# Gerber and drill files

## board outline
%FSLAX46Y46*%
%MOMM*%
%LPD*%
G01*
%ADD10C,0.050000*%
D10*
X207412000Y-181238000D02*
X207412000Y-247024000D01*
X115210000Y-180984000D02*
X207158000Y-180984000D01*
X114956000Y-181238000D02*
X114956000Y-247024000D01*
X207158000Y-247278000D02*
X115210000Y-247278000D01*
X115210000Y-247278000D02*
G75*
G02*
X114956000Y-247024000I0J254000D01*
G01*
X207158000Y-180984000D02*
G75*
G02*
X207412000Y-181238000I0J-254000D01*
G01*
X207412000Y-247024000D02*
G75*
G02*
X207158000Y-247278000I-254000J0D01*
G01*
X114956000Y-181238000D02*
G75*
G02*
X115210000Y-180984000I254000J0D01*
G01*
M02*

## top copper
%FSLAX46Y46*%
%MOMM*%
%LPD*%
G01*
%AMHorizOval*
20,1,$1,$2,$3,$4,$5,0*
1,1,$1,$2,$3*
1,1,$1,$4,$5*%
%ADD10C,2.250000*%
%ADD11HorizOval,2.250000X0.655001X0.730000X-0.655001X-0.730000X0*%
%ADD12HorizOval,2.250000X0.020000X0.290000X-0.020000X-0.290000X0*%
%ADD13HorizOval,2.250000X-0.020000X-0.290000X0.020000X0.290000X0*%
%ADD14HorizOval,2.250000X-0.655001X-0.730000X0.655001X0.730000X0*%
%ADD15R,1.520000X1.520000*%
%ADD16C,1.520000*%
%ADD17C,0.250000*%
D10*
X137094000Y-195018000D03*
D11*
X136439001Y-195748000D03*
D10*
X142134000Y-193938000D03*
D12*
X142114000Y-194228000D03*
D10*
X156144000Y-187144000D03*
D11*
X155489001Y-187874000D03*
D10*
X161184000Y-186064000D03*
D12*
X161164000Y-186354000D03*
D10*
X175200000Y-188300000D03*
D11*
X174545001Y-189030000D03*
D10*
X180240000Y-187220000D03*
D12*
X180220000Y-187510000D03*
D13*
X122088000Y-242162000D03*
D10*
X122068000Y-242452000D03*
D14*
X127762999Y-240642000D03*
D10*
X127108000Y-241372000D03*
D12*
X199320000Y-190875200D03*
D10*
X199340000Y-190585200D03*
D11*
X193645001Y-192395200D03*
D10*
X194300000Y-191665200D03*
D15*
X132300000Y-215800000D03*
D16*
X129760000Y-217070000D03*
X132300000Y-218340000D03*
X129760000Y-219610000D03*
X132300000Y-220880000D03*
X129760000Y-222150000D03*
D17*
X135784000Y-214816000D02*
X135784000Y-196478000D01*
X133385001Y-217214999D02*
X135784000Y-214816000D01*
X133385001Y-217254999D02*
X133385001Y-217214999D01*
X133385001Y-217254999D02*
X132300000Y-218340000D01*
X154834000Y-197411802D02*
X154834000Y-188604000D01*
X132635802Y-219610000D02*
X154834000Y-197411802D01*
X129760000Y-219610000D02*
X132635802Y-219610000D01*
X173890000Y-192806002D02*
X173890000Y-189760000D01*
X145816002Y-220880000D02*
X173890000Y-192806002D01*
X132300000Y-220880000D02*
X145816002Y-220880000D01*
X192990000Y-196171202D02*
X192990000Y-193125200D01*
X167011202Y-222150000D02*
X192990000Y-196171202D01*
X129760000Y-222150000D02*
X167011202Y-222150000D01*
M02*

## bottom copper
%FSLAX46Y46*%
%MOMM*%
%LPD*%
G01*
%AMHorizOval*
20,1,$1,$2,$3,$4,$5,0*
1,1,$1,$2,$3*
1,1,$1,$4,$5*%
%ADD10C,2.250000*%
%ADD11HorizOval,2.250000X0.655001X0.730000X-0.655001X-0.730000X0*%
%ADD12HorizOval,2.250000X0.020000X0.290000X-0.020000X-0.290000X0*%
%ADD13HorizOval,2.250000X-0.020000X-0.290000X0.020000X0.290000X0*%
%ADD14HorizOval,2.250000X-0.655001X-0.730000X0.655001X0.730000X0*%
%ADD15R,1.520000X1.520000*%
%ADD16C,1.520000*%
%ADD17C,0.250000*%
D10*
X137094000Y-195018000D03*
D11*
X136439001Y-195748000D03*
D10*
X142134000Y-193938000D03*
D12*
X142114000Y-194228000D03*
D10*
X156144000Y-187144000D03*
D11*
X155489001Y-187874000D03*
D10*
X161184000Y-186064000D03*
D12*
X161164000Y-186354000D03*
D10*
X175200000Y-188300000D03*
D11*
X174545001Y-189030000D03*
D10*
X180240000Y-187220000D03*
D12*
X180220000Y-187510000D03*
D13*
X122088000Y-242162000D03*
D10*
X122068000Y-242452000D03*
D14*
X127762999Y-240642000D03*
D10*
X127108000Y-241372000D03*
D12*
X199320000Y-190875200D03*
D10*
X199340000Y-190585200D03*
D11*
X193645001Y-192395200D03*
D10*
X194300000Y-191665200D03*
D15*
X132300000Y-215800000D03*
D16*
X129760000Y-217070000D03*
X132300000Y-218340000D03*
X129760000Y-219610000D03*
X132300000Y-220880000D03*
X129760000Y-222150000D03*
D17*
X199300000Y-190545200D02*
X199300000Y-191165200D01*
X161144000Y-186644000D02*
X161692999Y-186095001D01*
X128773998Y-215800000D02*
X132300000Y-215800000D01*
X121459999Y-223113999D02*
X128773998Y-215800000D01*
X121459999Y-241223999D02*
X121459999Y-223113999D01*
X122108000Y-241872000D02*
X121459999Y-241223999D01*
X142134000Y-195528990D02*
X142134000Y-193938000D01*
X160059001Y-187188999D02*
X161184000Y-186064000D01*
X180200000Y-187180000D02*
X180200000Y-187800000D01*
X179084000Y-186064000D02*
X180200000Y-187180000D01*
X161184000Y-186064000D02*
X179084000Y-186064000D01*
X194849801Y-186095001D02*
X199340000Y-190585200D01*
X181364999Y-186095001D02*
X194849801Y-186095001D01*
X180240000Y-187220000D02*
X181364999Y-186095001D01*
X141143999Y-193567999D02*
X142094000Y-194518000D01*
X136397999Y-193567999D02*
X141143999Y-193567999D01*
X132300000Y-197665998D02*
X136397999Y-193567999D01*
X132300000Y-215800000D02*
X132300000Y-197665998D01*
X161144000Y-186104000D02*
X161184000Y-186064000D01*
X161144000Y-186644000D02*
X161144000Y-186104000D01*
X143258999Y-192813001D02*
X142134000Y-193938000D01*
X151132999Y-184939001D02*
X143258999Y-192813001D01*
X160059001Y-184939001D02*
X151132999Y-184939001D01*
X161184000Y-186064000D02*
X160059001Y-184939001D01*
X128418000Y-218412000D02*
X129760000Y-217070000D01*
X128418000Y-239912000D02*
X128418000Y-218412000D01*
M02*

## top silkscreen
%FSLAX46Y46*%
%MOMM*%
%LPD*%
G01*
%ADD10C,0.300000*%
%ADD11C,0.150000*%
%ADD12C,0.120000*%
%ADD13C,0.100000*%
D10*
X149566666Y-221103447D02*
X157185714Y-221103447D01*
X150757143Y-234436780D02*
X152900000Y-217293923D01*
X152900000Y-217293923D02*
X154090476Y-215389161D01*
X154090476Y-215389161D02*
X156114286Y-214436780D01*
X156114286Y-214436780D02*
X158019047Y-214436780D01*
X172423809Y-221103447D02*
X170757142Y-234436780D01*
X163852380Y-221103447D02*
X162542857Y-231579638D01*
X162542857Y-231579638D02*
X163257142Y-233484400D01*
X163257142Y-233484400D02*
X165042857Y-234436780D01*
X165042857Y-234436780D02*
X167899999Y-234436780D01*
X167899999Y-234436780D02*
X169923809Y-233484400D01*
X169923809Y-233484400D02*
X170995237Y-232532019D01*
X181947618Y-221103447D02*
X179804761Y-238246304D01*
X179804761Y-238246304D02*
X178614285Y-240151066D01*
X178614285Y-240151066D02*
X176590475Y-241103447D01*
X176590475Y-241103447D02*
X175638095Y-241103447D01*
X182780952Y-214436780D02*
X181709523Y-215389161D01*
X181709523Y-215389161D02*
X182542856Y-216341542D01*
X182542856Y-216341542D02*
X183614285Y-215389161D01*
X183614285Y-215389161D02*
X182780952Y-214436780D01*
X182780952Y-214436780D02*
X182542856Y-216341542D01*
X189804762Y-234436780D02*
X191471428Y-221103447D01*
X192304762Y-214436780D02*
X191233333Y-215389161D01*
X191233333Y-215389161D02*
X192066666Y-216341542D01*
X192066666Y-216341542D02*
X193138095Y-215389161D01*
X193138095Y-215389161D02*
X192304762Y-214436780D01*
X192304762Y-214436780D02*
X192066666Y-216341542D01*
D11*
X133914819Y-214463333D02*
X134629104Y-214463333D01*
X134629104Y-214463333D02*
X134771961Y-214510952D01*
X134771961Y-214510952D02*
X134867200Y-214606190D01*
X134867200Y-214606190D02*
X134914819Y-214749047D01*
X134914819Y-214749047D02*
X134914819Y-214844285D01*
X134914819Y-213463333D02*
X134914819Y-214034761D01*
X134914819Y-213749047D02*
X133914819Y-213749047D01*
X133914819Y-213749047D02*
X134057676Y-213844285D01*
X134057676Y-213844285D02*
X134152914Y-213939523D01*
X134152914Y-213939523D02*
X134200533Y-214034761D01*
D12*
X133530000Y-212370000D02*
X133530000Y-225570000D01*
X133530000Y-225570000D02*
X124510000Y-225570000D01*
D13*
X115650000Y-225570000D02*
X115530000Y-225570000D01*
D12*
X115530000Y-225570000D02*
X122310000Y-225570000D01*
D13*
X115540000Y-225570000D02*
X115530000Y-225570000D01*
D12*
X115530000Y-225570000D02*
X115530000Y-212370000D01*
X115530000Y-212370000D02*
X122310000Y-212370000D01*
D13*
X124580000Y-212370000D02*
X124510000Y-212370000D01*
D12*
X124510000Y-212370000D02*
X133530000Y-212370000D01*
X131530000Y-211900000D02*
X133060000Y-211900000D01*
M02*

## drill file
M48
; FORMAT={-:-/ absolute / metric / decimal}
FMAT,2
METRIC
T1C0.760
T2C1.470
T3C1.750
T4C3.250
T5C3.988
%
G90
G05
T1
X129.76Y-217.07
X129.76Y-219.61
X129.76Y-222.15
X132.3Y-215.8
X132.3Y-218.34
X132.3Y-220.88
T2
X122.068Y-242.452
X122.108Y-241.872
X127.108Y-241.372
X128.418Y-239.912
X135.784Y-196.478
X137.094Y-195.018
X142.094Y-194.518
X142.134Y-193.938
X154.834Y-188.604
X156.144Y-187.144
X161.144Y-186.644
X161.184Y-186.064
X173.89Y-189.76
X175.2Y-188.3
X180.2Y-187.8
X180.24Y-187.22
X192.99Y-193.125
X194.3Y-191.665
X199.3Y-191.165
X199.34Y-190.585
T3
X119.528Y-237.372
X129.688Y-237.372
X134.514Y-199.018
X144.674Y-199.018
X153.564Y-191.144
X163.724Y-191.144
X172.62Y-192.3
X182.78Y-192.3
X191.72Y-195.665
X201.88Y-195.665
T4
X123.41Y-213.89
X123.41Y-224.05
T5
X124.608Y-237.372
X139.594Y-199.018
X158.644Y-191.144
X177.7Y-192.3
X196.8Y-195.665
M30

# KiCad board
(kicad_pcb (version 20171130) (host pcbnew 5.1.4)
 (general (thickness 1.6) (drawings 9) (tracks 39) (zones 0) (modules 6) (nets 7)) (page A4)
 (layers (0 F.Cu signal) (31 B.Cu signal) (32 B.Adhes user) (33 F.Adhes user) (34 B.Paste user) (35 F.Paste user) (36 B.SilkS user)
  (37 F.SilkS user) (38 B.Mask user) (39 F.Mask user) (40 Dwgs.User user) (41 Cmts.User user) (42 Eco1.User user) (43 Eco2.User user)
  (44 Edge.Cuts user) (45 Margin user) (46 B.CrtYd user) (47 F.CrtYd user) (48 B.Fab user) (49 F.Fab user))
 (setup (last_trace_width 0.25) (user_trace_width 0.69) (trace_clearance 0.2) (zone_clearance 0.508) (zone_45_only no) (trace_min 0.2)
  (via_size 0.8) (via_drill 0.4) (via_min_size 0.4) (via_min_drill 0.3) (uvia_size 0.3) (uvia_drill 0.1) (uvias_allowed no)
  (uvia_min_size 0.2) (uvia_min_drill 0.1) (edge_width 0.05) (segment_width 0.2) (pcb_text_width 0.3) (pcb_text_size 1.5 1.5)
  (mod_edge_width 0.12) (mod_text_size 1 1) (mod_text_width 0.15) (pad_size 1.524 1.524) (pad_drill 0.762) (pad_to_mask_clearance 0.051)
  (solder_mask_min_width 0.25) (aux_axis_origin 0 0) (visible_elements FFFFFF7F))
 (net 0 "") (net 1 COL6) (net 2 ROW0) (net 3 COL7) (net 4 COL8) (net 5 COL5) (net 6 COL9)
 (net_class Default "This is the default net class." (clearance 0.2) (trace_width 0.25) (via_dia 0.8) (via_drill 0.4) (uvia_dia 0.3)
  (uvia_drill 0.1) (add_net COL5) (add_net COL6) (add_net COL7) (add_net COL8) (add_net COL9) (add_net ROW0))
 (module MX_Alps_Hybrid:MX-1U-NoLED (layer F.Cu) (at 139.594 199.018)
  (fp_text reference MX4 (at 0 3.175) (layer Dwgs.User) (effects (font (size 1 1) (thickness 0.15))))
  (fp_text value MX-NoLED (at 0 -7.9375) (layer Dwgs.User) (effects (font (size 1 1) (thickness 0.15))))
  (pad "" np_thru_hole circle (at 5.08 0 48.0996) (size 1.75 1.75) (drill 1.75) (layers *.Cu *.Mask))
  (pad "" np_thru_hole circle (at -5.08 0 48.0996) (size 1.75 1.75) (drill 1.75) (layers *.Cu *.Mask))
  (pad 1 thru_hole circle (at -2.5 -4) (size 2.25 2.25) (drill 1.47) (layers *.Cu B.Mask) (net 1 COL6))
  (pad "" np_thru_hole circle (at 0 0) (size 3.9878 3.9878) (drill 3.9878) (layers *.Cu *.Mask))
  (pad 1 thru_hole oval (at -3.81 -2.54 48.0996) (size 4.211556 2.25) (drill 1.47 (offset 0.980778 0)) (layers *.Cu B.Mask) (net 1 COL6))
  (pad 2 thru_hole circle (at 2.54 -5.08) (size 2.25 2.25) (drill 1.47) (layers *.Cu B.Mask) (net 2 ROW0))
  (pad 2 thru_hole oval (at 2.5 -4.5 86.0548) (size 2.831378 2.25) (drill 1.47 (offset 0.290689 0)) (layers *.Cu B.Mask) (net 2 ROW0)))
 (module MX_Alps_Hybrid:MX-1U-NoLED (layer F.Cu) (at 158.644 191.144)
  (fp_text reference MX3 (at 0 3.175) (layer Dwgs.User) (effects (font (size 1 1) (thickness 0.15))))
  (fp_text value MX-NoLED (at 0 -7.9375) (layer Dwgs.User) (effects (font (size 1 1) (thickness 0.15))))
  (pad "" np_thru_hole circle (at 5.08 0 48.0996) (size 1.75 1.75) (drill 1.75) (layers *.Cu *.Mask))
  (pad "" np_thru_hole circle (at -5.08 0 48.0996) (size 1.75 1.75) (drill 1.75) (layers *.Cu *.Mask))
  (pad 1 thru_hole circle (at -2.5 -4) (size 2.25 2.25) (drill 1.47) (layers *.Cu B.Mask) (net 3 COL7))
  (pad "" np_thru_hole circle (at 0 0) (size 3.9878 3.9878) (drill 3.9878) (layers *.Cu *.Mask))
  (pad 1 thru_hole oval (at -3.81 -2.54 48.0996) (size 4.211556 2.25) (drill 1.47 (offset 0.980778 0)) (layers *.Cu B.Mask) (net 3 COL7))
  (pad 2 thru_hole circle (at 2.54 -5.08) (size 2.25 2.25) (drill 1.47) (layers *.Cu B.Mask) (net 2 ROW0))
  (pad 2 thru_hole oval (at 2.5 -4.5 86.0548) (size 2.831378 2.25) (drill 1.47 (offset 0.290689 0)) (layers *.Cu B.Mask) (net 2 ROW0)))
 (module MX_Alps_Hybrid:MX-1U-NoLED (layer F.Cu) (at 177.7 192.3)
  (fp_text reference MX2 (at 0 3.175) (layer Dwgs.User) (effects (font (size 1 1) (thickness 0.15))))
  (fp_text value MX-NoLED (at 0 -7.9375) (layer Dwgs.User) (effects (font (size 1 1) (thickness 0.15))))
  (pad "" np_thru_hole circle (at 5.08 0 48.0996) (size 1.75 1.75) (drill 1.75) (layers *.Cu *.Mask))
  (pad "" np_thru_hole circle (at -5.08 0 48.0996) (size 1.75 1.75) (drill 1.75) (layers *.Cu *.Mask))
  (pad 1 thru_hole circle (at -2.5 -4) (size 2.25 2.25) (drill 1.47) (layers *.Cu B.Mask) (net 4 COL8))
  (pad "" np_thru_hole circle (at 0 0) (size 3.9878 3.9878) (drill 3.9878) (layers *.Cu *.Mask))
  (pad 1 thru_hole oval (at -3.81 -2.54 48.0996) (size 4.211556 2.25) (drill 1.47 (offset 0.980778 0)) (layers *.Cu B.Mask) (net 4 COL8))
  (pad 2 thru_hole circle (at 2.54 -5.08) (size 2.25 2.25) (drill 1.47) (layers *.Cu B.Mask) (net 2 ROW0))
  (pad 2 thru_hole oval (at 2.5 -4.5 86.0548) (size 2.831378 2.25) (drill 1.47 (offset 0.290689 0)) (layers *.Cu B.Mask) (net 2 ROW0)))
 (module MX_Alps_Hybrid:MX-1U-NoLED (layer F.Cu) (at 124.608 237.372 180)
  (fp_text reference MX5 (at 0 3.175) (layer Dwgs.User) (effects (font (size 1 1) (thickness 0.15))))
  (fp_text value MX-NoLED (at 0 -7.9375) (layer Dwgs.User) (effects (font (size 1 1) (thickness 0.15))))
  (pad 2 thru_hole oval (at 2.5 -4.5 266.0548) (size 2.831378 2.25) (drill 1.47 (offset 0.290689 0)) (layers *.Cu B.Mask) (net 2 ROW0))
  (pad 2 thru_hole circle (at 2.54 -5.08 180) (size 2.25 2.25) (drill 1.47) (layers *.Cu B.Mask) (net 2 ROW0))
  (pad 1 thru_hole oval (at -3.81 -2.54 228.0996) (size 4.211556 2.25) (drill 1.47 (offset 0.980778 0)) (layers *.Cu B.Mask) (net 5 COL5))
  (pad "" np_thru_hole circle (at 0 0 180) (size 3.9878 3.9878) (drill 3.9878) (layers *.Cu *.Mask))
  (pad 1 thru_hole circle (at -2.5 -4 180) (size 2.25 2.25) (drill 1.47) (layers *.Cu B.Mask) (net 5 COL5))
  (pad "" np_thru_hole circle (at -5.08 0 228.0996) (size 1.75 1.75) (drill 1.75) (layers *.Cu *.Mask))
  (pad "" np_thru_hole circle (at 5.08 0 228.0996) (size 1.75 1.75) (drill 1.75) (layers *.Cu *.Mask)))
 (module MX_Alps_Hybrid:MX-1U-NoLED (layer F.Cu) (at 196.8 195.6652)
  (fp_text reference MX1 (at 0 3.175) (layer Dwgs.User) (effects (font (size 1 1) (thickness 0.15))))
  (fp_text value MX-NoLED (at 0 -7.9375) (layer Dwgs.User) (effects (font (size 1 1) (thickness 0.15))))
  (pad 2 thru_hole oval (at 2.5 -4.5 86.0548) (size 2.831378 2.25) (drill 1.47 (offset 0.290689 0)) (layers *.Cu B.Mask) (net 2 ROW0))
  (pad 2 thru_hole circle (at 2.54 -5.08) (size 2.25 2.25) (drill 1.47) (layers *.Cu B.Mask) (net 2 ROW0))
  (pad 1 thru_hole oval (at -3.81 -2.54 48.0996) (size 4.211556 2.25) (drill 1.47 (offset 0.980778 0)) (layers *.Cu B.Mask) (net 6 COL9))
  (pad "" np_thru_hole circle (at 0 0) (size 3.9878 3.9878) (drill 3.9878) (layers *.Cu *.Mask))
  (pad 1 thru_hole circle (at -2.5 -4) (size 2.25 2.25) (drill 1.47) (layers *.Cu B.Mask) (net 6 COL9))
  (pad "" np_thru_hole circle (at -5.08 0 48.0996) (size 1.75 1.75) (drill 1.75) (layers *.Cu *.Mask))
  (pad "" np_thru_hole circle (at 5.08 0 48.0996) (size 1.75 1.75) (drill 1.75) (layers *.Cu *.Mask)))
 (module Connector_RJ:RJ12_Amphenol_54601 (layer F.Cu) (at 132.3 215.8 270)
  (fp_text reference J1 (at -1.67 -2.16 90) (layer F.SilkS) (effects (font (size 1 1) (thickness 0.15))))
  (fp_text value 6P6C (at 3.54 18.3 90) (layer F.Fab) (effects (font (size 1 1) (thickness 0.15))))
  (fp_line (start -3.43 -1.23) (end 9.77 -1.23) (layer F.SilkS) (width 0.12))
  (fp_line (start 9.77 -1.23) (end 9.77 7.79) (layer F.SilkS) (width 0.12))
  (fp_line (start 9.77 16.65) (end 9.77 16.77) (layer F.SilkS) (width 0.1))
  (fp_line (start 9.77 16.77) (end 9.77 9.99) (layer F.SilkS) (width 0.12))
  (fp_line (start 9.77 16.76) (end 9.77 16.77) (layer F.SilkS) (width 0.1))
  (fp_line (start 9.77 16.77) (end -3.43 16.77) (layer F.SilkS) (width 0.12))
  (fp_line (start -3.43 16.77) (end -3.43 9.99) (layer F.SilkS) (width 0.12))
  (fp_line (start -3.43 7.72) (end -3.43 7.79) (layer F.SilkS) (width 0.1))
  (fp_line (start -3.43 7.79) (end -3.43 -1.23) (layer F.SilkS) (width 0.12))
  (fp_line (start -3.9 0.77) (end -3.9 -0.76) (layer F.SilkS) (width 0.12))
  (pad 1 thru_hole rect (at 0 0 270) (size 1.52 1.52) (drill 0.76) (layers *.Cu *.Mask) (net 2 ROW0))
  (pad "" np_thru_hole circle (at -1.91 8.89 270) (size 3.25 3.25) (drill 3.25) (layers *.Cu *.Mask))
  (pad 2 thru_hole circle (at 1.27 2.54 270) (size 1.52 1.52) (drill 0.76) (layers *.Cu *.Mask) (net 5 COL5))
  (pad 3 thru_hole circle (at 2.54 0 270) (size 1.52 1.52) (drill 0.76) (layers *.Cu *.Mask) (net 1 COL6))
  (pad 4 thru_hole circle (at 3.81 2.54 270) (size 1.52 1.52) (drill 0.76) (layers *.Cu *.Mask) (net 3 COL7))
  (pad 5 thru_hole circle (at 5.08 0 270) (size 1.52 1.52) (drill 0.76) (layers *.Cu *.Mask) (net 4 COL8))
  (pad 6 thru_hole circle (at 6.35 2.54 270) (size 1.52 1.52) (drill 0.76) (layers *.Cu *.Mask) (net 6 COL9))
  (pad "" np_thru_hole circle (at 8.25 8.89 270) (size 3.25 3.25) (drill 3.25) (layers *.Cu *.Mask)))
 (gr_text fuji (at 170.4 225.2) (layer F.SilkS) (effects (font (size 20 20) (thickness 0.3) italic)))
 (gr_line (start 207.412 181.238) (end 207.412 247.024) (layer Edge.Cuts) (width 0.05))
 (gr_line (start 115.21 180.984) (end 207.158 180.984) (layer Edge.Cuts) (width 0.05))
 (gr_line (start 114.956 181.238) (end 114.956 247.024) (layer Edge.Cuts) (width 0.05))
 (gr_line (start 207.158 247.278) (end 115.21 247.278) (layer Edge.Cuts) (width 0.05))
 (gr_arc (start 115.21 247.024) (end 115.21 247.278) (angle 90) (layer Edge.Cuts) (width 0.05))
 (gr_arc (start 207.158 181.238) (end 207.158 180.984) (angle 90) (layer Edge.Cuts) (width 0.05))
 (gr_arc (start 207.158 247.024) (end 207.412 247.024) (angle 90) (layer Edge.Cuts) (width 0.05))
 (gr_arc (start 115.21 181.238) (end 114.956 181.238) (angle 90) (layer Edge.Cuts) (width 0.05))
 (segment (start 199.3 190.5452) (end 199.3 191.1652) (width 0.25) (layer B.Cu) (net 2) (status 30))
 (segment (start 161.144 186.644) (end 161.692999 186.095001) (width 0.25) (layer B.Cu) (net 2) (status 30))
 (segment (start 128.773998 215.8) (end 132.3 215.8) (width 0.25) (layer B.Cu) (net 2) (status 20))
 (segment (start 121.459999 223.113999) (end 128.773998 215.8) (width 0.25) (layer B.Cu) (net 2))
 (segment (start 121.459999 241.223999) (end 121.459999 223.113999) (width 0.25) (layer B.Cu) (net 2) (status 10))
 (segment (start 122.108 241.872) (end 121.459999 241.223999) (width 0.25) (layer B.Cu) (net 2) (status 30))
 (segment (start 142.134 195.52899) (end 142.134 193.938) (width 0.25) (layer B.Cu) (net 2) (status 30))
 (segment (start 160.059001 187.188999) (end 161.184 186.064) (width 0.25) (layer B.Cu) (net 2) (status 30))
 (segment (start 180.2 187.18) (end 180.2 187.8) (width 0.25) (layer B.Cu) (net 2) (status 30))
 (segment (start 179.084 186.064) (end 180.2 187.18) (width 0.25) (layer B.Cu) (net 2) (status 20))
 (segment (start 161.184 186.064) (end 179.084 186.064) (width 0.25) (layer B.Cu) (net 2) (status 10))
 (segment (start 194.849801 186.095001) (end 199.34 190.5852) (width 0.25) (layer B.Cu) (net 2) (status 20))
 (segment (start 181.364999 186.095001) (end 194.849801 186.095001) (width 0.25) (layer B.Cu) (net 2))
 (segment (start 180.24 187.22) (end 181.364999 186.095001) (width 0.25) (layer B.Cu) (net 2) (status 10))
 (segment (start 141.143999 193.567999) (end 142.094 194.518) (width 0.25) (layer B.Cu) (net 2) (status 30))
 (segment (start 136.397999 193.567999) (end 141.143999 193.567999) (width 0.25) (layer B.Cu) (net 2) (status 20))
 (segment (start 132.3 197.665998) (end 136.397999 193.567999) (width 0.25) (layer B.Cu) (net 2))
 (segment (start 132.3 215.8) (end 132.3 197.665998) (width 0.25) (layer B.Cu) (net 2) (status 10))
 (segment (start 161.144 186.104) (end 161.184 186.064) (width 0.25) (layer B.Cu) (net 2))
 (segment (start 161.144 186.644) (end 161.144 186.104) (width 0.25) (layer B.Cu) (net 2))
 (segment (start 143.258999 192.813001) (end 142.134 193.938) (width 0.25) (layer B.Cu) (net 2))
 (segment (start 151.132999 184.939001) (end 143.258999 192.813001) (width 0.25) (layer B.Cu) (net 2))
 (segment (start 160.059001 184.939001) (end 151.132999 184.939001) (width 0.25) (layer B.Cu) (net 2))
 (segment (start 161.184 186.064) (end 160.059001 184.939001) (width 0.25) (layer B.Cu) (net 2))
 (segment (start 128.418 218.412) (end 129.76 217.07) (width 0.25) (layer B.Cu) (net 5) (status 20))
 (segment (start 128.418 239.912) (end 128.418 218.412) (width 0.25) (layer B.Cu) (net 5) (status 10))
 (segment (start 135.784 214.816) (end 135.784 196.478) (width 0.25) (layer F.Cu) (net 1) (status 20))
 (segment (start 133.385001 217.214999) (end 135.784 214.816) (width 0.25) (layer F.Cu) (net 1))
 (segment (start 133.385001 217.254999) (end 133.385001 217.214999) (width 0.25) (layer F.Cu) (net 1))
 (segment (start 133.385001 217.254999) (end 132.3 218.34) (width 0.25) (layer F.Cu) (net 1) (status 20))
 (segment (start 154.834 197.411802) (end 154.834 188.604) (width 0.25) (layer F.Cu) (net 3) (status 20))
 (segment (start 132.635802 219.61) (end 154.834 197.411802) (width 0.25) (layer F.Cu) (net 3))
 (segment (start 129.76 219.61) (end 132.635802 219.61) (width 0.25) (layer F.Cu) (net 3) (status 10))
 (segment (start 173.89 192.806002) (end 173.89 189.76) (width 0.25) (layer F.Cu) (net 4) (status 20))
 (segment (start 145.816002 220.88) (end 173.89 192.806002) (width 0.25) (layer F.Cu) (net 4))
 (segment (start 132.3 220.88) (end 145.816002 220.88) (width 0.25) (layer F.Cu) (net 4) (status 10))
 (segment (start 192.99 196.171202) (end 192.99 193.1252) (width 0.25) (layer F.Cu) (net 6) (status 20))
 (segment (start 167.011202 222.15) (end 192.99 196.171202) (width 0.25) (layer F.Cu) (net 6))
 (segment (start 129.76 222.15) (end 167.011202 222.15) (width 0.25) (layer F.Cu) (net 6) (status 10)))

